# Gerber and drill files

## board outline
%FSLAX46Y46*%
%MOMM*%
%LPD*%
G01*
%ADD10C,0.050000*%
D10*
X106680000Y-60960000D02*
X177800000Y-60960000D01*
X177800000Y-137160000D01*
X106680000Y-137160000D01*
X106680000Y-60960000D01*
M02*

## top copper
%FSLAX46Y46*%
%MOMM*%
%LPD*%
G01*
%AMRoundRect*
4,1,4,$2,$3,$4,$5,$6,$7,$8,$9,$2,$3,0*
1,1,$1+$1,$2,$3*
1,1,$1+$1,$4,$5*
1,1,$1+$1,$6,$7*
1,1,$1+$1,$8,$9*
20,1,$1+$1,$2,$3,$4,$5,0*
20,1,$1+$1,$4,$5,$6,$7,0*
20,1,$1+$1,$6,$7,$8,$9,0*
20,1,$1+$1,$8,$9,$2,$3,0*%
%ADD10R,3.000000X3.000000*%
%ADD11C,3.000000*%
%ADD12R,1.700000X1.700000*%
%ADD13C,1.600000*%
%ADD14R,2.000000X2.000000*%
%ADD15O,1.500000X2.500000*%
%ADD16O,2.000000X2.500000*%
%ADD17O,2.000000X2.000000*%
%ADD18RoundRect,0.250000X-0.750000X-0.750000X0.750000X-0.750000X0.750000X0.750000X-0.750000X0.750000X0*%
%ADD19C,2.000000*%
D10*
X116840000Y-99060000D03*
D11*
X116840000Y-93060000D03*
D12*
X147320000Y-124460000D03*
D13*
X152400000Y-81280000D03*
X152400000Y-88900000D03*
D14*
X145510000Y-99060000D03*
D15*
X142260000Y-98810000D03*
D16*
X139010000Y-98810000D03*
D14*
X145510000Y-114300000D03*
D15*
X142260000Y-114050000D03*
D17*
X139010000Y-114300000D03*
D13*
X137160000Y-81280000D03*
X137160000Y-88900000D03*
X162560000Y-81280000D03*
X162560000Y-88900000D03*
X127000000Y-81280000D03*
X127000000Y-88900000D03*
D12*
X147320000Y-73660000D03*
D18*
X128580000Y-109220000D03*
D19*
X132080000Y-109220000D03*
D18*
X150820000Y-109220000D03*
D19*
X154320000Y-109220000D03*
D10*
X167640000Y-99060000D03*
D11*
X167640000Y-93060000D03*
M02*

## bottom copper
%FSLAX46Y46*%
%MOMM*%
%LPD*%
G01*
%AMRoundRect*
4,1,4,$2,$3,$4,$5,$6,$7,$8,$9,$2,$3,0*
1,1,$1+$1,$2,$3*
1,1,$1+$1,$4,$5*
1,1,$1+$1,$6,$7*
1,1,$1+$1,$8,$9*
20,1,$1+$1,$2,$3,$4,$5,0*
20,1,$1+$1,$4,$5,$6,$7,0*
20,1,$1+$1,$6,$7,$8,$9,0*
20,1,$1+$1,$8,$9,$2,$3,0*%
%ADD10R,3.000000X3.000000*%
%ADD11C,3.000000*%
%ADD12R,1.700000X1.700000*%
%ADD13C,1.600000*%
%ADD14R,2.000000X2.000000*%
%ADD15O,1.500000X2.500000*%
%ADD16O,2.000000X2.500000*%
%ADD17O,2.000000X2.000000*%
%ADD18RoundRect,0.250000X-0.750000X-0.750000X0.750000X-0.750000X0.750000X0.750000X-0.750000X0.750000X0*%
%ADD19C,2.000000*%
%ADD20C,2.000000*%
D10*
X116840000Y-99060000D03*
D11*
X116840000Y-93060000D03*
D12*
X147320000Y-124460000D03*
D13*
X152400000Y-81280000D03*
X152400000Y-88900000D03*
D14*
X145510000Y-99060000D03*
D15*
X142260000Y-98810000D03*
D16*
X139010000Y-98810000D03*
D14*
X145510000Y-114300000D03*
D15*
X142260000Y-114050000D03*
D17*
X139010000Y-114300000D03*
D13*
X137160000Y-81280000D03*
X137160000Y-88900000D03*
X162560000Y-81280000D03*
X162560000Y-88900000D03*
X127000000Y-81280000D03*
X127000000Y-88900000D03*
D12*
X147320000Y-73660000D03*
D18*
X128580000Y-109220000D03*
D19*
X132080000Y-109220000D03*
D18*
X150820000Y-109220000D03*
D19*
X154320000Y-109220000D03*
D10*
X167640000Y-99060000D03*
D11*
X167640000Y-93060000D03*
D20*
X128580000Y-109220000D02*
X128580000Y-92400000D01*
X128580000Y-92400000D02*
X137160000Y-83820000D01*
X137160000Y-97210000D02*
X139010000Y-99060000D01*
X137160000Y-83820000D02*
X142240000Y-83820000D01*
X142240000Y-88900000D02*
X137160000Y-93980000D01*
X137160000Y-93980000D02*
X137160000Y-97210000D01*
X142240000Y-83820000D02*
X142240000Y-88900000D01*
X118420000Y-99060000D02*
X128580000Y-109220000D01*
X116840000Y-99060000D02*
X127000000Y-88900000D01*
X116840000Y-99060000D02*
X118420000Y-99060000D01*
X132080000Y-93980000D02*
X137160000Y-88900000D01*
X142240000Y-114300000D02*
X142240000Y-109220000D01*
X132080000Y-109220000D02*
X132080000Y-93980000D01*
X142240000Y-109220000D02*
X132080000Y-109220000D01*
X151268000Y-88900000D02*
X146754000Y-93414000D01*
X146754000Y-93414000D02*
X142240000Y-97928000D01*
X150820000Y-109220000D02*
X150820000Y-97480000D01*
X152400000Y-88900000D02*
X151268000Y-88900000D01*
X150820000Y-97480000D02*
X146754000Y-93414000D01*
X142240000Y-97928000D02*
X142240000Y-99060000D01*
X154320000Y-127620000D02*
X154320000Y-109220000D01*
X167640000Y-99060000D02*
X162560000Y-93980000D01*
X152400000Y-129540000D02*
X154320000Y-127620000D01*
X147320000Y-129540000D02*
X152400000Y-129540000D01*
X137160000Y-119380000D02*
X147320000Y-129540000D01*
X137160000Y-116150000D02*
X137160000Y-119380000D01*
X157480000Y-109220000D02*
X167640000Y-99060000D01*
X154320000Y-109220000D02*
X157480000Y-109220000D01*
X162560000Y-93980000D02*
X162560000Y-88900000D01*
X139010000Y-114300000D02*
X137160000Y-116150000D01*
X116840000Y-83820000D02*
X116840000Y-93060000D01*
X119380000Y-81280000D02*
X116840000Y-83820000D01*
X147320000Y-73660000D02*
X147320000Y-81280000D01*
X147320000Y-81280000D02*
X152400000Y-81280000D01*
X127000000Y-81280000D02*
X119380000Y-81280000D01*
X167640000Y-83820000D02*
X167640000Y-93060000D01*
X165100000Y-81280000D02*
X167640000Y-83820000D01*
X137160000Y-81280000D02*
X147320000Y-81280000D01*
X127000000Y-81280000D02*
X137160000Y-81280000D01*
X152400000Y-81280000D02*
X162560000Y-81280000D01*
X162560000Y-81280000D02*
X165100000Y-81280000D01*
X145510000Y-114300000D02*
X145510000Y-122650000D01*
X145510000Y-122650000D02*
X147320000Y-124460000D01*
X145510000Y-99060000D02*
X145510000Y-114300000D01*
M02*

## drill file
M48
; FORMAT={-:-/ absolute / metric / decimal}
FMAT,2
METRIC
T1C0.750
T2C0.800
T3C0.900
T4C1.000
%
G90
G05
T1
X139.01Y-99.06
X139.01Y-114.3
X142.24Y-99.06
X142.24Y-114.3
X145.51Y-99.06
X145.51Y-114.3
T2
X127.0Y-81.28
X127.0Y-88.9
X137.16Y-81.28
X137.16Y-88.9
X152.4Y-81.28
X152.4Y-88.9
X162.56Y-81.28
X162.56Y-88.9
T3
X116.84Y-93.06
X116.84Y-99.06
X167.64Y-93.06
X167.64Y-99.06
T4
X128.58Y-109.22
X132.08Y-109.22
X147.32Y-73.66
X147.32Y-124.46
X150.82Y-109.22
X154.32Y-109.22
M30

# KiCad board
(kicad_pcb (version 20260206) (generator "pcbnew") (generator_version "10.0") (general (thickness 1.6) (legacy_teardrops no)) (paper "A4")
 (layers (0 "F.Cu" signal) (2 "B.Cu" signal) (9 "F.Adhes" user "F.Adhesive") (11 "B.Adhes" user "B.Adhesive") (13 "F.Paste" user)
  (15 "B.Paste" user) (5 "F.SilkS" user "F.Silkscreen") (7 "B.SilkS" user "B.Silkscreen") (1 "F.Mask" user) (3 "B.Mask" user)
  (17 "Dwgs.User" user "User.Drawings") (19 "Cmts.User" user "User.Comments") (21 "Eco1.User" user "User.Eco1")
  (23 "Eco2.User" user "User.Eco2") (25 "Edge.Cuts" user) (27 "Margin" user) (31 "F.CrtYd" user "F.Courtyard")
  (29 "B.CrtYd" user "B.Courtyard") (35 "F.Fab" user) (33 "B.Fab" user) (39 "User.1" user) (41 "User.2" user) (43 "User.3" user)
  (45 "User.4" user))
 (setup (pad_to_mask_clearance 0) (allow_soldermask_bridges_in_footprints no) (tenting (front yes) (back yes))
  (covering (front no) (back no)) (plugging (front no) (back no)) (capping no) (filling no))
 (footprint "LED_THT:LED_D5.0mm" (layer "F.Cu") (at 116.84 99.06 90)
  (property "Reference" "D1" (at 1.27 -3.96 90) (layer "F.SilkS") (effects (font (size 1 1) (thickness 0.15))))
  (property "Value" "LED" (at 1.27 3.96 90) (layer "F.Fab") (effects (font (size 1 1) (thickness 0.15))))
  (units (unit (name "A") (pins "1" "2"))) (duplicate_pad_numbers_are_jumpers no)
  (pad "1" thru_hole rect (at 0 0 90) (size 3 3) (drill 0.9) (layers "*.Cu" "*.Mask") (remove_unused_layers no) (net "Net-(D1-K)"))
  (pad "2" thru_hole circle (at 6 0 90) (size 3 3) (drill 0.9) (layers "*.Cu" "*.Mask") (remove_unused_layers no) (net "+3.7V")))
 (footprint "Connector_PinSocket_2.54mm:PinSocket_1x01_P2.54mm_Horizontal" (layer "F.Cu") (at 147.32 124.46 90)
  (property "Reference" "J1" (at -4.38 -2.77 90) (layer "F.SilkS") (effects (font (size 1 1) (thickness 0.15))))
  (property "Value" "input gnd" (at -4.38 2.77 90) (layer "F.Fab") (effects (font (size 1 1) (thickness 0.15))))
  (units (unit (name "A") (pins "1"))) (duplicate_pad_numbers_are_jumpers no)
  (pad "1" thru_hole rect (at 0 0 90) (size 1.7 1.7) (drill 1) (layers "*.Cu" "*.Mask") (remove_unused_layers no) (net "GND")))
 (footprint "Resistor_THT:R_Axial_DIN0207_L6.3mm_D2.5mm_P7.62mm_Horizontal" (layer "F.Cu") (at 152.4 81.28 -90)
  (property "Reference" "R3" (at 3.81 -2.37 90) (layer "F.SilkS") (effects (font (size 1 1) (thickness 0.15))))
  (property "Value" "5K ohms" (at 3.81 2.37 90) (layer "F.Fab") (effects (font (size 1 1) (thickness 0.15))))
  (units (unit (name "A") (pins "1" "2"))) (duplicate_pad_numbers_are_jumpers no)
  (pad "1" thru_hole circle (at 0 0 270) (size 1.6 1.6) (drill 0.8) (layers "*.Cu" "*.Mask") (remove_unused_layers no) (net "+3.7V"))
  (pad "2" thru_hole circle (at 7.62 0 270) (size 1.6 1.6) (drill 0.8) (layers "*.Cu" "*.Mask") (remove_unused_layers no) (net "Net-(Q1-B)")))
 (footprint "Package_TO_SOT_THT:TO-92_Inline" (layer "F.Cu") (at 143.51 99.06 180)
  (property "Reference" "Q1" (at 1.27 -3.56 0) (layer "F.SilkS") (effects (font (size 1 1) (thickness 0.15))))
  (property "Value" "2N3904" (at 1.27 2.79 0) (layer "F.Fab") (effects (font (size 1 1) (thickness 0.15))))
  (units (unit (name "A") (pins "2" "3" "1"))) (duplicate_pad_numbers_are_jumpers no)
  (pad "1" thru_hole rect (at -2 0 180) (size 2 2) (drill 0.75) (layers "*.Cu" "*.Mask") (remove_unused_layers no) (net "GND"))
  (pad "2" thru_hole oval (at 1.27 0 180) (size 1.5 2.5) (drill 0.75 (offset -0.02 0.25)) (layers "*.Cu" "*.Mask") (remove_unused_layers no)
   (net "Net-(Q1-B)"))
  (pad "3" thru_hole oval (at 4.5 0 180) (size 2 2.5) (drill 0.75 (offset 0 0.25)) (layers "*.Cu" "*.Mask") (remove_unused_layers no)
   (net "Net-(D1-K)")))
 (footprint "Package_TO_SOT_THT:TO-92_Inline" (layer "F.Cu") (at 143.51 114.3 180)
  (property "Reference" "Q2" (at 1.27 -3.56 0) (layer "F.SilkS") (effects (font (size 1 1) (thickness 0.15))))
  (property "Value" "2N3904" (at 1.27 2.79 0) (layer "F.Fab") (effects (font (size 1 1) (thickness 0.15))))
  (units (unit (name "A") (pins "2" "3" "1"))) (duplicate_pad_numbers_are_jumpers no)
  (pad "1" thru_hole rect (at -2 0 180) (size 2 2) (drill 0.75) (layers "*.Cu" "*.Mask") (remove_unused_layers no) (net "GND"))
  (pad "2" thru_hole oval (at 1.27 0 180) (size 1.5 2.5) (drill 0.75 (offset -0.02 0.25)) (layers "*.Cu" "*.Mask") (remove_unused_layers no)
   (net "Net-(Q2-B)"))
  (pad "3" thru_hole oval (at 4.5 0 180) (size 2 2) (drill 0.75) (layers "*.Cu" "*.Mask") (remove_unused_layers no) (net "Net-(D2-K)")))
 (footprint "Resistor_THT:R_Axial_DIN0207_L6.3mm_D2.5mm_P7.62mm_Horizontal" (layer "F.Cu") (at 137.16 81.28 -90)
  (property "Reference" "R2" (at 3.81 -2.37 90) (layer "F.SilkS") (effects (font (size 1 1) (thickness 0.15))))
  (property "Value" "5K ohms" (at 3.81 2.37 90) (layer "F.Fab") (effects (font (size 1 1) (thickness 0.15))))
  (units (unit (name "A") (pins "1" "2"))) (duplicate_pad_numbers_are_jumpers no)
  (pad "1" thru_hole circle (at 0 0 270) (size 1.6 1.6) (drill 0.8) (layers "*.Cu" "*.Mask") (remove_unused_layers no) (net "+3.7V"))
  (pad "2" thru_hole circle (at 7.62 0 270) (size 1.6 1.6) (drill 0.8) (layers "*.Cu" "*.Mask") (remove_unused_layers no) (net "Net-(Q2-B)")))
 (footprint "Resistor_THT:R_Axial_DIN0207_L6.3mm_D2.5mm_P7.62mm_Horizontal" (layer "F.Cu") (at 162.56 81.28 -90)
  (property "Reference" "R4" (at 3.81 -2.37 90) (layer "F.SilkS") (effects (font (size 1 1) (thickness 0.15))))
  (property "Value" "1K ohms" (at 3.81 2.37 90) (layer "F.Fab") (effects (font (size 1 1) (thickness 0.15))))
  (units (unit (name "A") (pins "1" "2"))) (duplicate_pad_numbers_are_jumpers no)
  (pad "1" thru_hole circle (at 0 0 270) (size 1.6 1.6) (drill 0.8) (layers "*.Cu" "*.Mask") (remove_unused_layers no) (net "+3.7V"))
  (pad "2" thru_hole circle (at 7.62 0 270) (size 1.6 1.6) (drill 0.8) (layers "*.Cu" "*.Mask") (remove_unused_layers no) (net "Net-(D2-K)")))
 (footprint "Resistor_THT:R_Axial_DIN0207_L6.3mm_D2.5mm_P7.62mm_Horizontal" (layer "F.Cu") (at 127 81.28 -90)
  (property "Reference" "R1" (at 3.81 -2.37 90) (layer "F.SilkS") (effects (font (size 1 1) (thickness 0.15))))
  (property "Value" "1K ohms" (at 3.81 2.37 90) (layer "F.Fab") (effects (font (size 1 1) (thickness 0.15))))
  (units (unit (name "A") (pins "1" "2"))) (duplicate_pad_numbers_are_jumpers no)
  (pad "1" thru_hole circle (at 0 0 270) (size 1.6 1.6) (drill 0.8) (layers "*.Cu" "*.Mask") (remove_unused_layers no) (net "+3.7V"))
  (pad "2" thru_hole circle (at 7.62 0 270) (size 1.6 1.6) (drill 0.8) (layers "*.Cu" "*.Mask") (remove_unused_layers no) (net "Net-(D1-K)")))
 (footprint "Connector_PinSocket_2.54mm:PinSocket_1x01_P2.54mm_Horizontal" (layer "F.Cu") (at 147.32 73.66 -90)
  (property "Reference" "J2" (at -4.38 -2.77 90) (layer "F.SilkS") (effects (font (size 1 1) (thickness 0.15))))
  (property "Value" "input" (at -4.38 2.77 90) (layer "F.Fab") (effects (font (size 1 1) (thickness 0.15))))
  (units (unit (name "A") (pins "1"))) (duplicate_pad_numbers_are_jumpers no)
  (pad "1" thru_hole rect (at 0 0 270) (size 1.7 1.7) (drill 1) (layers "*.Cu" "*.Mask") (remove_unused_layers no) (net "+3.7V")))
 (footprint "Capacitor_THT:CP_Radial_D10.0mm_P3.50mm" (layer "F.Cu") (at 128.58 109.22)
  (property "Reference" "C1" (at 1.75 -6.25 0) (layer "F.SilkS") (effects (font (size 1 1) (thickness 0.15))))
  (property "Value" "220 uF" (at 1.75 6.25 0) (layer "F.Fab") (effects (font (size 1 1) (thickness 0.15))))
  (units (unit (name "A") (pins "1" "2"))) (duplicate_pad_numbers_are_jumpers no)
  (pad "1" thru_hole roundrect (at 0 0) (size 2 2) (drill 1) (layers "*.Cu" "*.Mask") (remove_unused_layers no) (roundrect_rratio 0.125)
   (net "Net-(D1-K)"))
  (pad "2" thru_hole circle (at 3.5 0) (size 2 2) (drill 1) (layers "*.Cu" "*.Mask") (remove_unused_layers no) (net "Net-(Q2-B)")))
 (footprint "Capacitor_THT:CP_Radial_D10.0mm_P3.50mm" (layer "F.Cu") (at 150.82 109.22)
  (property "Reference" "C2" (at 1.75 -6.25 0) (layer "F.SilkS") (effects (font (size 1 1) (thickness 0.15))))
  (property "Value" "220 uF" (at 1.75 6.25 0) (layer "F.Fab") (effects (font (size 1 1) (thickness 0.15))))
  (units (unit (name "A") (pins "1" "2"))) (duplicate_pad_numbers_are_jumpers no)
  (pad "1" thru_hole roundrect (at 0 0) (size 2 2) (drill 1) (layers "*.Cu" "*.Mask") (remove_unused_layers no) (roundrect_rratio 0.125)
   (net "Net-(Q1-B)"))
  (pad "2" thru_hole circle (at 3.5 0) (size 2 2) (drill 1) (layers "*.Cu" "*.Mask") (remove_unused_layers no) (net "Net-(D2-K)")))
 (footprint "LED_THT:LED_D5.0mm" (layer "F.Cu") (at 167.64 99.06 90)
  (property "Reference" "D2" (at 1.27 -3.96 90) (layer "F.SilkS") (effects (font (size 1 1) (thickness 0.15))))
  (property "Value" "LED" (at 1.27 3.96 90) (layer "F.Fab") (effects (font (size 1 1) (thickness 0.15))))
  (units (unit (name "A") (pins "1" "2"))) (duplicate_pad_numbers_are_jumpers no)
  (pad "1" thru_hole rect (at 0 0 90) (size 3 3) (drill 0.9) (layers "*.Cu" "*.Mask") (remove_unused_layers no) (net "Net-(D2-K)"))
  (pad "2" thru_hole circle (at 6 0 90) (size 3 3) (drill 0.9) (layers "*.Cu" "*.Mask") (remove_unused_layers no) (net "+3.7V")))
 (gr_rect (start 106.68 60.96) (end 177.8 137.16) (stroke (width 0.05) (type default)) (fill no) (layer "Edge.Cuts"))
 (segment (start 128.58 109.22) (end 128.58 92.4) (width 2) (layer "B.Cu") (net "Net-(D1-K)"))
 (segment (start 128.58 92.4) (end 137.16 83.82) (width 2) (layer "B.Cu") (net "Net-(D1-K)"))
 (segment (start 137.16 97.21) (end 139.01 99.06) (width 2) (layer "B.Cu") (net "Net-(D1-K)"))
 (segment (start 137.16 83.82) (end 142.24 83.82) (width 2) (layer "B.Cu") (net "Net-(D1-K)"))
 (segment (start 142.24 88.9) (end 137.16 93.98) (width 2) (layer "B.Cu") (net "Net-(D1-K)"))
 (segment (start 137.16 93.98) (end 137.16 97.21) (width 2) (layer "B.Cu") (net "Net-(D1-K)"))
 (segment (start 142.24 83.82) (end 142.24 88.9) (width 2) (layer "B.Cu") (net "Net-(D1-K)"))
 (segment (start 118.42 99.06) (end 128.58 109.22) (width 2) (layer "B.Cu") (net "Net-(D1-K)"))
 (segment (start 116.84 99.06) (end 127 88.9) (width 2) (layer "B.Cu") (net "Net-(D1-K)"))
 (segment (start 116.84 99.06) (end 118.42 99.06) (width 2) (layer "B.Cu") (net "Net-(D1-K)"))
 (segment (start 132.08 93.98) (end 137.16 88.9) (width 2) (layer "B.Cu") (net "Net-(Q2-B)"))
 (segment (start 142.24 114.3) (end 142.24 109.22) (width 2) (layer "B.Cu") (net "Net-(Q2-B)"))
 (segment (start 132.08 109.22) (end 132.08 93.98) (width 2) (layer "B.Cu") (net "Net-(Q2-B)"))
 (segment (start 142.24 109.22) (end 132.08 109.22) (width 2) (layer "B.Cu") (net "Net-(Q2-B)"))
 (segment (start 151.268 88.9) (end 146.754 93.414) (width 2) (layer "B.Cu") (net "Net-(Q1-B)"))
 (segment (start 146.754 93.414) (end 142.24 97.928) (width 2) (layer "B.Cu") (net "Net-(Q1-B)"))
 (segment (start 150.82 109.22) (end 150.82 97.48) (width 2) (layer "B.Cu") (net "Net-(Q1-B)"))
 (segment (start 152.4 88.9) (end 151.268 88.9) (width 2) (layer "B.Cu") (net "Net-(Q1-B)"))
 (segment (start 150.82 97.48) (end 146.754 93.414) (width 2) (layer "B.Cu") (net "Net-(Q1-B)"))
 (segment (start 142.24 97.928) (end 142.24 99.06) (width 2) (layer "B.Cu") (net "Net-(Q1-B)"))
 (segment (start 154.32 127.62) (end 154.32 109.22) (width 2) (layer "B.Cu") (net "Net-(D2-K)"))
 (segment (start 167.64 99.06) (end 162.56 93.98) (width 2) (layer "B.Cu") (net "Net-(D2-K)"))
 (segment (start 152.4 129.54) (end 154.32 127.62) (width 2) (layer "B.Cu") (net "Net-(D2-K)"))
 (segment (start 147.32 129.54) (end 152.4 129.54) (width 2) (layer "B.Cu") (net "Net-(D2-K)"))
 (segment (start 137.16 119.38) (end 147.32 129.54) (width 2) (layer "B.Cu") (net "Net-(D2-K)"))
 (segment (start 137.16 116.15) (end 137.16 119.38) (width 2) (layer "B.Cu") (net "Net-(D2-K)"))
 (segment (start 157.48 109.22) (end 167.64 99.06) (width 2) (layer "B.Cu") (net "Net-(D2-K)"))
 (segment (start 154.32 109.22) (end 157.48 109.22) (width 2) (layer "B.Cu") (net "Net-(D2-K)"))
 (segment (start 162.56 93.98) (end 162.56 88.9) (width 2) (layer "B.Cu") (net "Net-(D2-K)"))
 (segment (start 139.01 114.3) (end 137.16 116.15) (width 2) (layer "B.Cu") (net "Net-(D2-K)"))
 (segment (start 116.84 83.82) (end 116.84 93.06) (width 2) (layer "B.Cu") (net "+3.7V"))
 (segment (start 119.38 81.28) (end 116.84 83.82) (width 2) (layer "B.Cu") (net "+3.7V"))
 (segment (start 147.32 73.66) (end 147.32 81.28) (width 2) (layer "B.Cu") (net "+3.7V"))
 (segment (start 147.32 81.28) (end 152.4 81.28) (width 2) (layer "B.Cu") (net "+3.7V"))
 (segment (start 127 81.28) (end 119.38 81.28) (width 2) (layer "B.Cu") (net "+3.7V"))
 (segment (start 167.64 83.82) (end 167.64 93.06) (width 2) (layer "B.Cu") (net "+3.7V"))
 (segment (start 165.1 81.28) (end 167.64 83.82) (width 2) (layer "B.Cu") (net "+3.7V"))
 (segment (start 137.16 81.28) (end 147.32 81.28) (width 2) (layer "B.Cu") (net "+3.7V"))
 (segment (start 127 81.28) (end 137.16 81.28) (width 2) (layer "B.Cu") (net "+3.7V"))
 (segment (start 152.4 81.28) (end 162.56 81.28) (width 2) (layer "B.Cu") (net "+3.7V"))
 (segment (start 162.56 81.28) (end 165.1 81.28) (width 2) (layer "B.Cu") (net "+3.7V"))
 (segment (start 145.51 114.3) (end 145.51 122.65) (width 2) (layer "B.Cu") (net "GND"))
 (segment (start 145.51 122.65) (end 147.32 124.46) (width 2) (layer "B.Cu") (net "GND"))
 (segment (start 145.51 99.06) (end 145.51 114.3) (width 2) (layer "B.Cu") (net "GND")))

